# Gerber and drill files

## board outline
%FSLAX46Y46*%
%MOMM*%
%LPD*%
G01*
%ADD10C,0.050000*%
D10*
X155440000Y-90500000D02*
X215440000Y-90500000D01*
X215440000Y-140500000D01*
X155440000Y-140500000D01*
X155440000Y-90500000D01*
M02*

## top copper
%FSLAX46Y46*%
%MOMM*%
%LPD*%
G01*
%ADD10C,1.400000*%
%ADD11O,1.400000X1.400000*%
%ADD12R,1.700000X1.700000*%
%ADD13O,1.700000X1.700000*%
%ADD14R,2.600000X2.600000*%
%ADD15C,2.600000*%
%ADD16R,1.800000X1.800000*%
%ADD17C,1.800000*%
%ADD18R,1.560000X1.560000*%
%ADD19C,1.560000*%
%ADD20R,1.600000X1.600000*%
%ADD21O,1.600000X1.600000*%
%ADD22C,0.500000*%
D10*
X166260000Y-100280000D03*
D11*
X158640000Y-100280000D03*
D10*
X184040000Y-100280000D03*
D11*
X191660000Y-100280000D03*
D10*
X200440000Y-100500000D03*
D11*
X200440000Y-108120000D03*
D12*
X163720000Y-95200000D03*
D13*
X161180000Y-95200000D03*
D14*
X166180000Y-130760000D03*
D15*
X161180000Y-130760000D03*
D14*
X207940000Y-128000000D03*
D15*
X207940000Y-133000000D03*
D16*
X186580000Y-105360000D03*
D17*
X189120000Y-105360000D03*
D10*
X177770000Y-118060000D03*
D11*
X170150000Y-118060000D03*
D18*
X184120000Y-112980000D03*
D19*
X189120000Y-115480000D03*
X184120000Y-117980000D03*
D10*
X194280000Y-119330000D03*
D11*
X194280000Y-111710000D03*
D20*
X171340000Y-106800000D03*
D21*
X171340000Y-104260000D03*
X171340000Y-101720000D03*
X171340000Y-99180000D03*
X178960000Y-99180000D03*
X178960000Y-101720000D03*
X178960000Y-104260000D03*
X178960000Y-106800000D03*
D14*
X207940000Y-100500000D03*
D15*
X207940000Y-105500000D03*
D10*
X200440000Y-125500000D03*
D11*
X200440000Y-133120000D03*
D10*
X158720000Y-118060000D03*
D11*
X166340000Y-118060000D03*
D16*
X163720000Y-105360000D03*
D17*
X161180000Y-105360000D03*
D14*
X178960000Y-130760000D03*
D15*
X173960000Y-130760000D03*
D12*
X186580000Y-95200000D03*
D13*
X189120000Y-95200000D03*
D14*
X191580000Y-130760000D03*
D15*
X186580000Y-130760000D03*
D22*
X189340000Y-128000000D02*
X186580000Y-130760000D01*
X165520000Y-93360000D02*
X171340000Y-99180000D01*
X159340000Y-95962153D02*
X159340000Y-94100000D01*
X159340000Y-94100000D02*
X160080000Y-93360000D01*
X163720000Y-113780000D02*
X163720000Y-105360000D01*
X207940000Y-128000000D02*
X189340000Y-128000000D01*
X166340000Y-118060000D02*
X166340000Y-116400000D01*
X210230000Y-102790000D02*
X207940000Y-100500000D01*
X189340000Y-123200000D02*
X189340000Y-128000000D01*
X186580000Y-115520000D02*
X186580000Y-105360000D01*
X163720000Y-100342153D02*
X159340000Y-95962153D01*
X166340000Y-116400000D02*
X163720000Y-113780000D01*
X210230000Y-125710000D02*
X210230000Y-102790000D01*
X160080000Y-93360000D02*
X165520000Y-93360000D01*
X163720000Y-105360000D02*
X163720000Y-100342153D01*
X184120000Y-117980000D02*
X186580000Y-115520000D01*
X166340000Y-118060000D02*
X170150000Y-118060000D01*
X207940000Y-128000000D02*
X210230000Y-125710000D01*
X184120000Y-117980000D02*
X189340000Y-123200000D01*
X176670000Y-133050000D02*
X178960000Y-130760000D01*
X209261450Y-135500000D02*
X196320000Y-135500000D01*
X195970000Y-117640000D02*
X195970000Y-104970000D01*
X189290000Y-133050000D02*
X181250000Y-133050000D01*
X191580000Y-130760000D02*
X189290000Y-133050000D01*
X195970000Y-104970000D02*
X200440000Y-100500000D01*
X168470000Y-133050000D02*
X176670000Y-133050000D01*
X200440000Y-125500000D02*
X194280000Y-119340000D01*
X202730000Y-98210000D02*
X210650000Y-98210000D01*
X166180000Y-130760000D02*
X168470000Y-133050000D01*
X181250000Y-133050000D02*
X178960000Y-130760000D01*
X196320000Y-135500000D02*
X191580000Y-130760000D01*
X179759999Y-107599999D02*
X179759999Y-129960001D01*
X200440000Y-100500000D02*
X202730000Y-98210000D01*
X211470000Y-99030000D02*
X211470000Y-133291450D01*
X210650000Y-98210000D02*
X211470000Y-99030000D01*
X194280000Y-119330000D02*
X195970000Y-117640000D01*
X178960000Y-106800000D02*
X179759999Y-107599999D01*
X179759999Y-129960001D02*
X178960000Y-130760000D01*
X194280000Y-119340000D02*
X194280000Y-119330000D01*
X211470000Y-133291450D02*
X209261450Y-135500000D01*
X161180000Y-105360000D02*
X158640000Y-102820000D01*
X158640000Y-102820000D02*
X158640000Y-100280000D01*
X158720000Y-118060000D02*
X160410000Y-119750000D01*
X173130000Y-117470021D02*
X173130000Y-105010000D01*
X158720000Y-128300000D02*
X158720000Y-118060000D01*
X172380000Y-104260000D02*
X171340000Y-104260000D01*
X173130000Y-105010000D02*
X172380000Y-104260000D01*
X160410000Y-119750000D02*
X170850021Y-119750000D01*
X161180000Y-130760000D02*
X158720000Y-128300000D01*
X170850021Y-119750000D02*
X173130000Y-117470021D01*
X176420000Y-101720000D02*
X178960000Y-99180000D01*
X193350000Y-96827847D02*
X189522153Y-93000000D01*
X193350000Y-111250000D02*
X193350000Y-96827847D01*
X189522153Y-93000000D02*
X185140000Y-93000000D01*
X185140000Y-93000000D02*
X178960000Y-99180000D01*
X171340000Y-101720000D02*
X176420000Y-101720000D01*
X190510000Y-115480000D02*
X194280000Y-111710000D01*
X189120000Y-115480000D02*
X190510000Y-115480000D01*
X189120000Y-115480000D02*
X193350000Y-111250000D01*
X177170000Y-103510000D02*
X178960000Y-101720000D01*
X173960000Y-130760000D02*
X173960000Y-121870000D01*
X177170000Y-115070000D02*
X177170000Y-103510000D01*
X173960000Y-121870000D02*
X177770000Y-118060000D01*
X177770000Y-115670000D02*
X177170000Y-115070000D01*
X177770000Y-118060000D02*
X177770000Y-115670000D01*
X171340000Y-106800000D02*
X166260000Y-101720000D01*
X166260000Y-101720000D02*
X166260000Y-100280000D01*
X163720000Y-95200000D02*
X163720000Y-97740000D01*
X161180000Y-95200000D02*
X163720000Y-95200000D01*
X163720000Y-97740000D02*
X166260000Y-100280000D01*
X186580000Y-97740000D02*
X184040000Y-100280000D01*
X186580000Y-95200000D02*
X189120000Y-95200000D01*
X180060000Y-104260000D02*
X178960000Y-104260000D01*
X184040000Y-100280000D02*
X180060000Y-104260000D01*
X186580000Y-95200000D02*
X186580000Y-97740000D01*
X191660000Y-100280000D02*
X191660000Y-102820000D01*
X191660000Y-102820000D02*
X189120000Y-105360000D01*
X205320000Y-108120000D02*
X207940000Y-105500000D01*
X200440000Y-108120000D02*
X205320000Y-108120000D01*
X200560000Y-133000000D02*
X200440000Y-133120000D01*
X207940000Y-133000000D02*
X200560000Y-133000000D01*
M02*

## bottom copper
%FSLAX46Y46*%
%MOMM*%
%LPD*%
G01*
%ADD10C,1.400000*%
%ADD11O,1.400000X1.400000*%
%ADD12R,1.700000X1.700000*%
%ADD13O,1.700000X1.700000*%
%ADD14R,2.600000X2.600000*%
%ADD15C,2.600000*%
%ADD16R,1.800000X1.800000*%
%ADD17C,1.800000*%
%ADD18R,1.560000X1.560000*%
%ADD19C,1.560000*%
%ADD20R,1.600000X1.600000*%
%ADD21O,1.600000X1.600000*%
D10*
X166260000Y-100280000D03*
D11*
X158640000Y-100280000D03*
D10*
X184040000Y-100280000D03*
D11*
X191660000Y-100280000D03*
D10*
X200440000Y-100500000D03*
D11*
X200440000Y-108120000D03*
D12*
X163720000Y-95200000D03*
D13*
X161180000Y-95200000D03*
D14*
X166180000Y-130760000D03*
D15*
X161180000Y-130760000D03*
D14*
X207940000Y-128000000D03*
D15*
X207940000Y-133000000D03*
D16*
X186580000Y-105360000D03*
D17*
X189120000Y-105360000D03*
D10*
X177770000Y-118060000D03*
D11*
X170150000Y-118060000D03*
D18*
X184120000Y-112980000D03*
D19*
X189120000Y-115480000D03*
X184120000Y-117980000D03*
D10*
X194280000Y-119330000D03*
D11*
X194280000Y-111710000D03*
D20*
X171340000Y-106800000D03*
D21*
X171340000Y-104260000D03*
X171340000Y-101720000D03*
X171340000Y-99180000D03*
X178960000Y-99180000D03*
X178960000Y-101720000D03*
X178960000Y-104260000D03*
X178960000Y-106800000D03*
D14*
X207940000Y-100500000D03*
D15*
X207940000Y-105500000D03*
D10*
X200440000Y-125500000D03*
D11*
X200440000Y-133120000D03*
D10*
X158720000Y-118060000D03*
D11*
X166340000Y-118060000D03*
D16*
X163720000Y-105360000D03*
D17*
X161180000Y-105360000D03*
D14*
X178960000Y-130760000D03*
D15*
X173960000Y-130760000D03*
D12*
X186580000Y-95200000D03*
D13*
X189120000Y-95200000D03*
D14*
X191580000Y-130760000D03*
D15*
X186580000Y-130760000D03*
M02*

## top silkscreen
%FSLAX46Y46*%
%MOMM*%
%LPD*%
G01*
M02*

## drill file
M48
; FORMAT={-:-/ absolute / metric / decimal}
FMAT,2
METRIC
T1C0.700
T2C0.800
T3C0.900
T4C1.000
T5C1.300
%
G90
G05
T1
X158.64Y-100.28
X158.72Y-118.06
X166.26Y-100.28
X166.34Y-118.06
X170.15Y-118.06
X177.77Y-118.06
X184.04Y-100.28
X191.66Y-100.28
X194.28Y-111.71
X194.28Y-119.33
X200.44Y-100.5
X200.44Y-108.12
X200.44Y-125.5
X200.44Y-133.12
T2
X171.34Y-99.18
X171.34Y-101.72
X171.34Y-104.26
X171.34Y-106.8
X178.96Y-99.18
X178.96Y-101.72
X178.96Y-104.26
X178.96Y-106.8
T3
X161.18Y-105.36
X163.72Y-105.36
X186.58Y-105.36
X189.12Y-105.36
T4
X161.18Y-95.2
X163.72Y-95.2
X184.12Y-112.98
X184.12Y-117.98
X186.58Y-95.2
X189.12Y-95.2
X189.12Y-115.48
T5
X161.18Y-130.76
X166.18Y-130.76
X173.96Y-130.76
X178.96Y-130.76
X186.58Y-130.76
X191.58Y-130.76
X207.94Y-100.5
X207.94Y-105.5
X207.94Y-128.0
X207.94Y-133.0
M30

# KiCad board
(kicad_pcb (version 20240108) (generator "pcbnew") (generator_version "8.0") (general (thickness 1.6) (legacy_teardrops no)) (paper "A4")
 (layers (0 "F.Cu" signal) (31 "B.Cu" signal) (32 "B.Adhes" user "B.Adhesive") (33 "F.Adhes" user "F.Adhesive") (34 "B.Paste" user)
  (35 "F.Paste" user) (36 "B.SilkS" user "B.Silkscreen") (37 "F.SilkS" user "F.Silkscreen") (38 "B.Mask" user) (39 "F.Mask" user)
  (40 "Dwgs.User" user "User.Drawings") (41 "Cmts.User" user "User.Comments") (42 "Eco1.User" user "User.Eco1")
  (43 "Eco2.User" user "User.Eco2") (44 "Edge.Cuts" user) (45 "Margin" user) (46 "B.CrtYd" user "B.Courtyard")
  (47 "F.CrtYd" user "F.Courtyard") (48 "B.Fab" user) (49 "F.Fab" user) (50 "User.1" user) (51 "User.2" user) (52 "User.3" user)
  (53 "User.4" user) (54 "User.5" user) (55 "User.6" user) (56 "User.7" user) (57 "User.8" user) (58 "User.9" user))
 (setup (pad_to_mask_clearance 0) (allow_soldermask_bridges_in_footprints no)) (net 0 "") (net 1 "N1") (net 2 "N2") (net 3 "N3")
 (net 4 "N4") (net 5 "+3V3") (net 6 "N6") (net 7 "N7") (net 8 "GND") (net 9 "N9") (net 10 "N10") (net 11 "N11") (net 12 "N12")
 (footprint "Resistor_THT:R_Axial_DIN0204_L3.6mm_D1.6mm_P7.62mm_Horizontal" (layer "B.Cu") (at 166.26 100.28 180)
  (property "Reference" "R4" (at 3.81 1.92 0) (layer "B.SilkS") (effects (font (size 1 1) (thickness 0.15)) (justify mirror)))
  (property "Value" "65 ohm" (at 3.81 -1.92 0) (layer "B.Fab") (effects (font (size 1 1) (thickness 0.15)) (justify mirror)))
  (pad "1" thru_hole circle (at 0 0 180) (size 1.4 1.4) (drill 0.7) (layers "*.Cu" "*.Mask") (remove_unused_layers no) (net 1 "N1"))
  (pad "2" thru_hole oval (at 7.62 0 180) (size 1.4 1.4) (drill 0.7) (layers "*.Cu" "*.Mask") (remove_unused_layers no) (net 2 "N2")))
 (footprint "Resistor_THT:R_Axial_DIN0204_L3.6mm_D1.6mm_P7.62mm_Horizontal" (layer "B.Cu") (at 184.04 100.28)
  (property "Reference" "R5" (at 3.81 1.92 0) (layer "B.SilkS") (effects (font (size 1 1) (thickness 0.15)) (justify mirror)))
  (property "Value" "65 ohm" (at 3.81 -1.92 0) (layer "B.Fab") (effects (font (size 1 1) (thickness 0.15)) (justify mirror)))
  (pad "1" thru_hole circle (at 0 0) (size 1.4 1.4) (drill 0.7) (layers "*.Cu" "*.Mask") (remove_unused_layers no) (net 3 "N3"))
  (pad "2" thru_hole oval (at 7.62 0) (size 1.4 1.4) (drill 0.7) (layers "*.Cu" "*.Mask") (remove_unused_layers no) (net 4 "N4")))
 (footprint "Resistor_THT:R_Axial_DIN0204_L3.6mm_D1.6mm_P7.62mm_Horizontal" (layer "B.Cu") (at 200.44 100.5 -90)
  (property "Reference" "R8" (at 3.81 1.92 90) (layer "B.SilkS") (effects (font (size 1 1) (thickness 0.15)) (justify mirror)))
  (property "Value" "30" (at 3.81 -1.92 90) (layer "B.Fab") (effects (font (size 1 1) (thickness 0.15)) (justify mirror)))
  (pad "1" thru_hole circle (at 0 0 270) (size 1.4 1.4) (drill 0.7) (layers "*.Cu" "*.Mask") (remove_unused_layers no) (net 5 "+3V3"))
  (pad "2" thru_hole oval (at 7.62 0 270) (size 1.4 1.4) (drill 0.7) (layers "*.Cu" "*.Mask") (remove_unused_layers no) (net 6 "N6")))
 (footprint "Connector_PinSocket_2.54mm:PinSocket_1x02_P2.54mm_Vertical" (layer "B.Cu") (at 163.72 95.2 90)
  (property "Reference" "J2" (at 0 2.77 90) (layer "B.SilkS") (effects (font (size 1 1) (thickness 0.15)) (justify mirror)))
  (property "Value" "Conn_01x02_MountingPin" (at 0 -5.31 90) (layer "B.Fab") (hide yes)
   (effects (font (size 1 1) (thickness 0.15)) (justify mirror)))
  (pad "1" thru_hole rect (at 0 0 90) (size 1.7 1.7) (drill 1) (layers "*.Cu" "*.Mask") (remove_unused_layers no) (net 1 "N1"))
  (pad "2" thru_hole oval (at 0 -2.54 90) (size 1.7 1.7) (drill 1) (layers "*.Cu" "*.Mask") (remove_unused_layers no) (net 1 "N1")))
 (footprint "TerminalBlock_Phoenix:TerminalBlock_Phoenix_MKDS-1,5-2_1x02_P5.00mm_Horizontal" (layer "B.Cu") (at 166.18 130.76 180)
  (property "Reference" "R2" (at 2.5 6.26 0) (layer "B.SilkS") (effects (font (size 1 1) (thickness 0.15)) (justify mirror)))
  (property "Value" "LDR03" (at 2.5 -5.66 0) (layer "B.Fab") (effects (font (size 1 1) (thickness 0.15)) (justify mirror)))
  (pad "1" thru_hole rect (at 0 0 180) (size 2.6 2.6) (drill 1.3) (layers "*.Cu" "*.Mask") (remove_unused_layers no) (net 5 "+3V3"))
  (pad "2" thru_hole circle (at 5 0 180) (size 2.6 2.6) (drill 1.3) (layers "*.Cu" "*.Mask") (remove_unused_layers no) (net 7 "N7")))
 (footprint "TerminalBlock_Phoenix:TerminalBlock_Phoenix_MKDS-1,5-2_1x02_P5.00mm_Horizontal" (layer "B.Cu") (at 207.94 128 -90)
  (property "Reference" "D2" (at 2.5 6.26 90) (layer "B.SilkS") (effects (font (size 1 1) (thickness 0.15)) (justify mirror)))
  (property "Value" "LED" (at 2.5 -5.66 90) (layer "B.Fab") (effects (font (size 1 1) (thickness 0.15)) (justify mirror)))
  (pad "1" thru_hole rect (at 0 0 270) (size 2.6 2.6) (drill 1.3) (layers "*.Cu" "*.Mask") (remove_unused_layers no) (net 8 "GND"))
  (pad "2" thru_hole circle (at 5 0 270) (size 2.6 2.6) (drill 1.3) (layers "*.Cu" "*.Mask") (remove_unused_layers no) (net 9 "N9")))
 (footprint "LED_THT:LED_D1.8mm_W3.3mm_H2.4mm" (layer "B.Cu") (at 186.58 105.36)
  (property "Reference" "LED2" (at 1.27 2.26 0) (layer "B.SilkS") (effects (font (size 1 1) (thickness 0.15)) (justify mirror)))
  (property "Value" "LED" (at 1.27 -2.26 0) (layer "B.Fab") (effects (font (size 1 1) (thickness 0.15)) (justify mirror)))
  (pad "1" thru_hole rect (at 0 0) (size 1.8 1.8) (drill 0.9) (layers "*.Cu" "*.Mask") (remove_unused_layers no) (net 8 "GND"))
  (pad "2" thru_hole circle (at 2.54 0) (size 1.8 1.8) (drill 0.9) (layers "*.Cu" "*.Mask") (remove_unused_layers no) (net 4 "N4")))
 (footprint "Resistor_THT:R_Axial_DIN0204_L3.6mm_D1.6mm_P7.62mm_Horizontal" (layer "B.Cu") (at 177.77 118.06 180)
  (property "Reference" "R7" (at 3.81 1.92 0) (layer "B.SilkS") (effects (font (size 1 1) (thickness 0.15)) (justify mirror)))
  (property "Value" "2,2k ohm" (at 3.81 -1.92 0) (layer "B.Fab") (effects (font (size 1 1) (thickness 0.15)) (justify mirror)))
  (pad "1" thru_hole circle (at 0 0 180) (size 1.4 1.4) (drill 0.7) (layers "*.Cu" "*.Mask") (remove_unused_layers no) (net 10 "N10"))
  (pad "2" thru_hole oval (at 7.62 0 180) (size 1.4 1.4) (drill 0.7) (layers "*.Cu" "*.Mask") (remove_unused_layers no) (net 8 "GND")))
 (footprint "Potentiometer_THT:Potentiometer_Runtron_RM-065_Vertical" (layer "B.Cu") (at 184.12 112.98 -90)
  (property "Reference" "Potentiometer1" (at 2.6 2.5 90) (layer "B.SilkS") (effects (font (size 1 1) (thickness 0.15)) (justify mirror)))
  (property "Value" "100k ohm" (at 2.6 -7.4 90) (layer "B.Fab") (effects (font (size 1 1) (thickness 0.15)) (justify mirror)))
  (pad "1" thru_hole rect (at 0 0 270) (size 1.56 1.56) (drill 1) (layers "*.Cu" "*.Mask") (remove_unused_layers no) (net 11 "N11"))
  (pad "2" thru_hole circle (at 2.5 -5 270) (size 1.56 1.56) (drill 1) (layers "*.Cu" "*.Mask") (remove_unused_layers no) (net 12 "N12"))
  (pad "3" thru_hole circle (at 5 0 270) (size 1.56 1.56) (drill 1) (layers "*.Cu" "*.Mask") (remove_unused_layers no) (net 8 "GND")))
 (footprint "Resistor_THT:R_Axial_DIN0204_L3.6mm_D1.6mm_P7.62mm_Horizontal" (layer "B.Cu") (at 194.28 119.33 90)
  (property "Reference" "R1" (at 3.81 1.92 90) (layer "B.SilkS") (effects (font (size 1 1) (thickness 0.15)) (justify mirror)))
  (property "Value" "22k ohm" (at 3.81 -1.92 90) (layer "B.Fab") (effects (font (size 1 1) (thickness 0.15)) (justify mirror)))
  (pad "1" thru_hole circle (at 0 0 90) (size 1.4 1.4) (drill 0.7) (layers "*.Cu" "*.Mask") (remove_unused_layers no) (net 5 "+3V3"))
  (pad "2" thru_hole oval (at 7.62 0 90) (size 1.4 1.4) (drill 0.7) (layers "*.Cu" "*.Mask") (remove_unused_layers no) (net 12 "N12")))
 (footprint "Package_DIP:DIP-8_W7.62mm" (layer "B.Cu") (at 171.34 106.8)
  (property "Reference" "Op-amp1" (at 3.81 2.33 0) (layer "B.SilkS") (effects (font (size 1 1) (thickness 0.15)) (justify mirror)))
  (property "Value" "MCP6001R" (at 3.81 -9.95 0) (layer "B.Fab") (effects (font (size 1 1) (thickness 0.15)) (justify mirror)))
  (pad "1" thru_hole rect (at 0 0) (size 1.6 1.6) (drill 0.8) (layers "*.Cu" "*.Mask") (remove_unused_layers no) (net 1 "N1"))
  (pad "2" thru_hole oval (at 0 -2.54) (size 1.6 1.6) (drill 0.8) (layers "*.Cu" "*.Mask") (remove_unused_layers no) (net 7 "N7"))
  (pad "3" thru_hole oval (at 0 -5.08) (size 1.6 1.6) (drill 0.8) (layers "*.Cu" "*.Mask") (remove_unused_layers no) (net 12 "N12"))
  (pad "4" thru_hole oval (at 0 -7.62) (size 1.6 1.6) (drill 0.8) (layers "*.Cu" "*.Mask") (remove_unused_layers no) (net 8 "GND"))
  (pad "5" thru_hole oval (at 7.62 -7.62) (size 1.6 1.6) (drill 0.8) (layers "*.Cu" "*.Mask") (remove_unused_layers no) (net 12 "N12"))
  (pad "6" thru_hole oval (at 7.62 -5.08) (size 1.6 1.6) (drill 0.8) (layers "*.Cu" "*.Mask") (remove_unused_layers no) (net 10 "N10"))
  (pad "7" thru_hole oval (at 7.62 -2.54) (size 1.6 1.6) (drill 0.8) (layers "*.Cu" "*.Mask") (remove_unused_layers no) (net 3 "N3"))
  (pad "8" thru_hole oval (at 7.62 0) (size 1.6 1.6) (drill 0.8) (layers "*.Cu" "*.Mask") (remove_unused_layers no) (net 5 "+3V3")))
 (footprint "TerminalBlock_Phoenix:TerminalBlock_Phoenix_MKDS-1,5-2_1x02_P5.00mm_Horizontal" (layer "B.Cu") (at 207.94 100.5 -90)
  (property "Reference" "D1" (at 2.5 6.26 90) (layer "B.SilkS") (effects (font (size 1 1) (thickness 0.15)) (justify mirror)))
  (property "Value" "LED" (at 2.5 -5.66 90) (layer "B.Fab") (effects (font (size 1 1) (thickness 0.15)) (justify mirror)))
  (pad "1" thru_hole rect (at 0 0 270) (size 2.6 2.6) (drill 1.3) (layers "*.Cu" "*.Mask") (remove_unused_layers no) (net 8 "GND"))
  (pad "2" thru_hole circle (at 5 0 270) (size 2.6 2.6) (drill 1.3) (layers "*.Cu" "*.Mask") (remove_unused_layers no) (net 6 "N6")))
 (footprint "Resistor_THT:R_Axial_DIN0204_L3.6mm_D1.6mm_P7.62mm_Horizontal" (layer "B.Cu") (at 200.44 125.5 -90)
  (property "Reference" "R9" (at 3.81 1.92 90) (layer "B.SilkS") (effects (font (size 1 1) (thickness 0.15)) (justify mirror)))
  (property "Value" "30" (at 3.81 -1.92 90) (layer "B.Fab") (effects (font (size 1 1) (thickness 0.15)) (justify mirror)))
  (pad "1" thru_hole circle (at 0 0 270) (size 1.4 1.4) (drill 0.7) (layers "*.Cu" "*.Mask") (remove_unused_layers no) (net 5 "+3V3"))
  (pad "2" thru_hole oval (at 7.62 0 270) (size 1.4 1.4) (drill 0.7) (layers "*.Cu" "*.Mask") (remove_unused_layers no) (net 9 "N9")))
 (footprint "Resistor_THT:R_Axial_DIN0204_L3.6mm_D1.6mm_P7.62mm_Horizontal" (layer "B.Cu") (at 158.72 118.06)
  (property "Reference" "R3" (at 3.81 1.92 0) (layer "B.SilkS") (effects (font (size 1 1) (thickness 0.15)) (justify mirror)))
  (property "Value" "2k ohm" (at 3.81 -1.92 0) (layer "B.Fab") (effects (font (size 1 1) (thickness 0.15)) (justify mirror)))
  (pad "1" thru_hole circle (at 0 0) (size 1.4 1.4) (drill 0.7) (layers "*.Cu" "*.Mask") (remove_unused_layers no) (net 7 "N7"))
  (pad "2" thru_hole oval (at 7.62 0) (size 1.4 1.4) (drill 0.7) (layers "*.Cu" "*.Mask") (remove_unused_layers no) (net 8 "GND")))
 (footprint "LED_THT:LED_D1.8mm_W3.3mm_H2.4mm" (layer "B.Cu") (at 163.72 105.36 180)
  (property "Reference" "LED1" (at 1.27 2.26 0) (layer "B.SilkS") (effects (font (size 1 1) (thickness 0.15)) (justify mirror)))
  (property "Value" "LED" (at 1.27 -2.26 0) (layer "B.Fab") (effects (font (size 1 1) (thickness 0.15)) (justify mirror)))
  (pad "1" thru_hole rect (at 0 0 180) (size 1.8 1.8) (drill 0.9) (layers "*.Cu" "*.Mask") (remove_unused_layers no) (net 8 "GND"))
  (pad "2" thru_hole circle (at 2.54 0 180) (size 1.8 1.8) (drill 0.9) (layers "*.Cu" "*.Mask") (remove_unused_layers no) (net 2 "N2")))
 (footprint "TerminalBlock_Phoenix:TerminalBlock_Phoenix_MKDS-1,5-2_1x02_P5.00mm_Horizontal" (layer "B.Cu") (at 178.96 130.76 180)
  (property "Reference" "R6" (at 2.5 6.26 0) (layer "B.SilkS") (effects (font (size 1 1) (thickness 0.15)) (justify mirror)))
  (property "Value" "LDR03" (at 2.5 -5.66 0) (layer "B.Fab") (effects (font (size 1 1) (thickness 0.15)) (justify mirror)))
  (pad "1" thru_hole rect (at 0 0 180) (size 2.6 2.6) (drill 1.3) (layers "*.Cu" "*.Mask") (remove_unused_layers no) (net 5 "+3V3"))
  (pad "2" thru_hole circle (at 5 0 180) (size 2.6 2.6) (drill 1.3) (layers "*.Cu" "*.Mask") (remove_unused_layers no) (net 10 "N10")))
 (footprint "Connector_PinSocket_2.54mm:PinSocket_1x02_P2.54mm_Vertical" (layer "B.Cu") (at 186.58 95.2 -90)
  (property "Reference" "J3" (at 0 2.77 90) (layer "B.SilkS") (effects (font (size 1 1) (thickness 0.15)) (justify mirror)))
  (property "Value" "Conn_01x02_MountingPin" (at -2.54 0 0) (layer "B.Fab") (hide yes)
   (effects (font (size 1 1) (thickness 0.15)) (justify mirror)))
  (pad "1" thru_hole rect (at 0 0 270) (size 1.7 1.7) (drill 1) (layers "*.Cu" "*.Mask") (remove_unused_layers no) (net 3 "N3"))
  (pad "2" thru_hole oval (at 0 -2.54 270) (size 1.7 1.7) (drill 1) (layers "*.Cu" "*.Mask") (remove_unused_layers no) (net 3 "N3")))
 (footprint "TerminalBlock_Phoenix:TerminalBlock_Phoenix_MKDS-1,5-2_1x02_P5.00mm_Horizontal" (layer "B.Cu") (at 191.58 130.76 180)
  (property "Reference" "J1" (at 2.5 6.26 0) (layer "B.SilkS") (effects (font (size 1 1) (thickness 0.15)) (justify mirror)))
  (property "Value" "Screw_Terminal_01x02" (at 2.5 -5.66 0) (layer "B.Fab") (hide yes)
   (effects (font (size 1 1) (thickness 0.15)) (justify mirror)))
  (pad "1" thru_hole rect (at 0 0 180) (size 2.6 2.6) (drill 1.3) (layers "*.Cu" "*.Mask") (remove_unused_layers no) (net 5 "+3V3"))
  (pad "2" thru_hole circle (at 5 0 180) (size 2.6 2.6) (drill 1.3) (layers "*.Cu" "*.Mask") (remove_unused_layers no) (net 8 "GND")))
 (gr_rect (start 155.44 90.5) (end 215.44 140.5) (stroke (width 0.05) (type default)) (fill none) (layer "Edge.Cuts"))
 (segment (start 189.34 128) (end 186.58 130.76) (width 0.5) (layer "F.Cu") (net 8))
 (segment (start 165.52 93.36) (end 171.34 99.18) (width 0.5) (layer "F.Cu") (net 8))
 (segment (start 159.34 95.962153) (end 159.34 94.1) (width 0.5) (layer "F.Cu") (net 8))
 (segment (start 159.34 94.1) (end 160.08 93.36) (width 0.5) (layer "F.Cu") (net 8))
 (segment (start 163.72 113.78) (end 163.72 105.36) (width 0.5) (layer "F.Cu") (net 8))
 (segment (start 207.94 128) (end 189.34 128) (width 0.5) (layer "F.Cu") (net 8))
 (segment (start 166.34 118.06) (end 166.34 116.4) (width 0.5) (layer "F.Cu") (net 8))
 (segment (start 210.23 102.79) (end 207.94 100.5) (width 0.5) (layer "F.Cu") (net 8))
 (segment (start 189.34 123.2) (end 189.34 128) (width 0.5) (layer "F.Cu") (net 8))
 (segment (start 186.58 115.52) (end 186.58 105.36) (width 0.5) (layer "F.Cu") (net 8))
 (segment (start 163.72 100.342153) (end 159.34 95.962153) (width 0.5) (layer "F.Cu") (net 8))
 (segment (start 166.34 116.4) (end 163.72 113.78) (width 0.5) (layer "F.Cu") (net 8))
 (segment (start 210.23 125.71) (end 210.23 102.79) (width 0.5) (layer "F.Cu") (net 8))
 (segment (start 160.08 93.36) (end 165.52 93.36) (width 0.5) (layer "F.Cu") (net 8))
 (segment (start 163.72 105.36) (end 163.72 100.342153) (width 0.5) (layer "F.Cu") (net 8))
 (segment (start 184.12 117.98) (end 186.58 115.52) (width 0.5) (layer "F.Cu") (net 8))
 (segment (start 166.34 118.06) (end 170.15 118.06) (width 0.5) (layer "F.Cu") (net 8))
 (segment (start 207.94 128) (end 210.23 125.71) (width 0.5) (layer "F.Cu") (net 8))
 (segment (start 184.12 117.98) (end 189.34 123.2) (width 0.5) (layer "F.Cu") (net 8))
 (segment (start 176.67 133.05) (end 178.96 130.76) (width 0.5) (layer "F.Cu") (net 5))
 (segment (start 209.26145 135.5) (end 196.32 135.5) (width 0.5) (layer "F.Cu") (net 5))
 (segment (start 195.97 117.64) (end 195.97 104.97) (width 0.5) (layer "F.Cu") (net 5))
 (segment (start 189.29 133.05) (end 181.25 133.05) (width 0.5) (layer "F.Cu") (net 5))
 (segment (start 191.58 130.76) (end 189.29 133.05) (width 0.5) (layer "F.Cu") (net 5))
 (segment (start 195.97 104.97) (end 200.44 100.5) (width 0.5) (layer "F.Cu") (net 5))
 (segment (start 168.47 133.05) (end 176.67 133.05) (width 0.5) (layer "F.Cu") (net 5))
 (segment (start 200.44 125.5) (end 194.28 119.34) (width 0.5) (layer "F.Cu") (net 5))
 (segment (start 202.73 98.21) (end 210.65 98.21) (width 0.5) (layer "F.Cu") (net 5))
 (segment (start 166.18 130.76) (end 168.47 133.05) (width 0.5) (layer "F.Cu") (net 5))
 (segment (start 181.25 133.05) (end 178.96 130.76) (width 0.5) (layer "F.Cu") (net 5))
 (segment (start 196.32 135.5) (end 191.58 130.76) (width 0.5) (layer "F.Cu") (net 5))
 (segment (start 179.759999 107.599999) (end 179.759999 129.960001) (width 0.5) (layer "F.Cu") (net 5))
 (segment (start 200.44 100.5) (end 202.73 98.21) (width 0.5) (layer "F.Cu") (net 5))
 (segment (start 211.47 99.03) (end 211.47 133.29145) (width 0.5) (layer "F.Cu") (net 5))
 (segment (start 210.65 98.21) (end 211.47 99.03) (width 0.5) (layer "F.Cu") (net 5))
 (segment (start 194.28 119.33) (end 195.97 117.64) (width 0.5) (layer "F.Cu") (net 5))
 (segment (start 178.96 106.8) (end 179.759999 107.599999) (width 0.5) (layer "F.Cu") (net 5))
 (segment (start 179.759999 129.960001) (end 178.96 130.76) (width 0.5) (layer "F.Cu") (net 5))
 (segment (start 194.28 119.34) (end 194.28 119.33) (width 0.5) (layer "F.Cu") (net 5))
 (segment (start 211.47 133.29145) (end 209.26145 135.5) (width 0.5) (layer "F.Cu") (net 5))
 (segment (start 161.18 105.36) (end 158.64 102.82) (width 0.5) (layer "F.Cu") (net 2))
 (segment (start 158.64 102.82) (end 158.64 100.28) (width 0.5) (layer "F.Cu") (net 2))
 (segment (start 158.72 118.06) (end 160.41 119.75) (width 0.5) (layer "F.Cu") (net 7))
 (segment (start 173.13 117.470021) (end 173.13 105.01) (width 0.5) (layer "F.Cu") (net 7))
 (segment (start 158.72 128.3) (end 158.72 118.06) (width 0.5) (layer "F.Cu") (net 7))
 (segment (start 172.38 104.26) (end 171.34 104.26) (width 0.5) (layer "F.Cu") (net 7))
 (segment (start 173.13 105.01) (end 172.38 104.26) (width 0.5) (layer "F.Cu") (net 7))
 (segment (start 160.41 119.75) (end 170.850021 119.75) (width 0.5) (layer "F.Cu") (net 7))
 (segment (start 161.18 130.76) (end 158.72 128.3) (width 0.5) (layer "F.Cu") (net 7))
 (segment (start 170.850021 119.75) (end 173.13 117.470021) (width 0.5) (layer "F.Cu") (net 7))
 (segment (start 176.42 101.72) (end 178.96 99.18) (width 0.5) (layer "F.Cu") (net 12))
 (segment (start 193.35 96.827847) (end 189.522153 93) (width 0.5) (layer "F.Cu") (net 12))
 (segment (start 193.35 111.25) (end 193.35 96.827847) (width 0.5) (layer "F.Cu") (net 12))
 (segment (start 189.522153 93) (end 185.14 93) (width 0.5) (layer "F.Cu") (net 12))
 (segment (start 185.14 93) (end 178.96 99.18) (width 0.5) (layer "F.Cu") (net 12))
 (segment (start 171.34 101.72) (end 176.42 101.72) (width 0.5) (layer "F.Cu") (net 12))
 (segment (start 190.51 115.48) (end 194.28 111.71) (width 0.5) (layer "F.Cu") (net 12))
 (segment (start 189.12 115.48) (end 190.51 115.48) (width 0.5) (layer "F.Cu") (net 12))
 (segment (start 189.12 115.48) (end 193.35 111.25) (width 0.5) (layer "F.Cu") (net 12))
 (segment (start 177.17 103.51) (end 178.96 101.72) (width 0.5) (layer "F.Cu") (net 10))
 (segment (start 173.96 130.76) (end 173.96 121.87) (width 0.5) (layer "F.Cu") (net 10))
 (segment (start 177.17 115.07) (end 177.17 103.51) (width 0.5) (layer "F.Cu") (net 10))
 (segment (start 173.96 121.87) (end 177.77 118.06) (width 0.5) (layer "F.Cu") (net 10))
 (segment (start 177.77 115.67) (end 177.17 115.07) (width 0.5) (layer "F.Cu") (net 10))
 (segment (start 177.77 118.06) (end 177.77 115.67) (width 0.5) (layer "F.Cu") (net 10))
 (segment (start 171.34 106.8) (end 166.26 101.72) (width 0.5) (layer "F.Cu") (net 1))
 (segment (start 166.26 101.72) (end 166.26 100.28) (width 0.5) (layer "F.Cu") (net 1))
 (segment (start 163.72 95.2) (end 163.72 97.74) (width 0.5) (layer "F.Cu") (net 1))
 (segment (start 161.18 95.2) (end 163.72 95.2) (width 0.5) (layer "F.Cu") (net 1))
 (segment (start 163.72 97.74) (end 166.26 100.28) (width 0.5) (layer "F.Cu") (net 1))
 (segment (start 186.58 97.74) (end 184.04 100.28) (width 0.5) (layer "F.Cu") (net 3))
 (segment (start 186.58 95.2) (end 189.12 95.2) (width 0.5) (layer "F.Cu") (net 3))
 (segment (start 180.06 104.26) (end 178.96 104.26) (width 0.5) (layer "F.Cu") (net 3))
 (segment (start 184.04 100.28) (end 180.06 104.26) (width 0.5) (layer "F.Cu") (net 3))
 (segment (start 186.58 95.2) (end 186.58 97.74) (width 0.5) (layer "F.Cu") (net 3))
 (segment (start 191.66 100.28) (end 191.66 102.82) (width 0.5) (layer "F.Cu") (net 4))
 (segment (start 191.66 102.82) (end 189.12 105.36) (width 0.5) (layer "F.Cu") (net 4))
 (segment (start 205.32 108.12) (end 207.94 105.5) (width 0.5) (layer "F.Cu") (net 6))
 (segment (start 200.44 108.12) (end 205.32 108.12) (width 0.5) (layer "F.Cu") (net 6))
 (segment (start 200.56 133) (end 200.44 133.12) (width 0.5) (layer "F.Cu") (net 9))
 (segment (start 207.94 133) (end 200.56 133) (width 0.5) (layer "F.Cu") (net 9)))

